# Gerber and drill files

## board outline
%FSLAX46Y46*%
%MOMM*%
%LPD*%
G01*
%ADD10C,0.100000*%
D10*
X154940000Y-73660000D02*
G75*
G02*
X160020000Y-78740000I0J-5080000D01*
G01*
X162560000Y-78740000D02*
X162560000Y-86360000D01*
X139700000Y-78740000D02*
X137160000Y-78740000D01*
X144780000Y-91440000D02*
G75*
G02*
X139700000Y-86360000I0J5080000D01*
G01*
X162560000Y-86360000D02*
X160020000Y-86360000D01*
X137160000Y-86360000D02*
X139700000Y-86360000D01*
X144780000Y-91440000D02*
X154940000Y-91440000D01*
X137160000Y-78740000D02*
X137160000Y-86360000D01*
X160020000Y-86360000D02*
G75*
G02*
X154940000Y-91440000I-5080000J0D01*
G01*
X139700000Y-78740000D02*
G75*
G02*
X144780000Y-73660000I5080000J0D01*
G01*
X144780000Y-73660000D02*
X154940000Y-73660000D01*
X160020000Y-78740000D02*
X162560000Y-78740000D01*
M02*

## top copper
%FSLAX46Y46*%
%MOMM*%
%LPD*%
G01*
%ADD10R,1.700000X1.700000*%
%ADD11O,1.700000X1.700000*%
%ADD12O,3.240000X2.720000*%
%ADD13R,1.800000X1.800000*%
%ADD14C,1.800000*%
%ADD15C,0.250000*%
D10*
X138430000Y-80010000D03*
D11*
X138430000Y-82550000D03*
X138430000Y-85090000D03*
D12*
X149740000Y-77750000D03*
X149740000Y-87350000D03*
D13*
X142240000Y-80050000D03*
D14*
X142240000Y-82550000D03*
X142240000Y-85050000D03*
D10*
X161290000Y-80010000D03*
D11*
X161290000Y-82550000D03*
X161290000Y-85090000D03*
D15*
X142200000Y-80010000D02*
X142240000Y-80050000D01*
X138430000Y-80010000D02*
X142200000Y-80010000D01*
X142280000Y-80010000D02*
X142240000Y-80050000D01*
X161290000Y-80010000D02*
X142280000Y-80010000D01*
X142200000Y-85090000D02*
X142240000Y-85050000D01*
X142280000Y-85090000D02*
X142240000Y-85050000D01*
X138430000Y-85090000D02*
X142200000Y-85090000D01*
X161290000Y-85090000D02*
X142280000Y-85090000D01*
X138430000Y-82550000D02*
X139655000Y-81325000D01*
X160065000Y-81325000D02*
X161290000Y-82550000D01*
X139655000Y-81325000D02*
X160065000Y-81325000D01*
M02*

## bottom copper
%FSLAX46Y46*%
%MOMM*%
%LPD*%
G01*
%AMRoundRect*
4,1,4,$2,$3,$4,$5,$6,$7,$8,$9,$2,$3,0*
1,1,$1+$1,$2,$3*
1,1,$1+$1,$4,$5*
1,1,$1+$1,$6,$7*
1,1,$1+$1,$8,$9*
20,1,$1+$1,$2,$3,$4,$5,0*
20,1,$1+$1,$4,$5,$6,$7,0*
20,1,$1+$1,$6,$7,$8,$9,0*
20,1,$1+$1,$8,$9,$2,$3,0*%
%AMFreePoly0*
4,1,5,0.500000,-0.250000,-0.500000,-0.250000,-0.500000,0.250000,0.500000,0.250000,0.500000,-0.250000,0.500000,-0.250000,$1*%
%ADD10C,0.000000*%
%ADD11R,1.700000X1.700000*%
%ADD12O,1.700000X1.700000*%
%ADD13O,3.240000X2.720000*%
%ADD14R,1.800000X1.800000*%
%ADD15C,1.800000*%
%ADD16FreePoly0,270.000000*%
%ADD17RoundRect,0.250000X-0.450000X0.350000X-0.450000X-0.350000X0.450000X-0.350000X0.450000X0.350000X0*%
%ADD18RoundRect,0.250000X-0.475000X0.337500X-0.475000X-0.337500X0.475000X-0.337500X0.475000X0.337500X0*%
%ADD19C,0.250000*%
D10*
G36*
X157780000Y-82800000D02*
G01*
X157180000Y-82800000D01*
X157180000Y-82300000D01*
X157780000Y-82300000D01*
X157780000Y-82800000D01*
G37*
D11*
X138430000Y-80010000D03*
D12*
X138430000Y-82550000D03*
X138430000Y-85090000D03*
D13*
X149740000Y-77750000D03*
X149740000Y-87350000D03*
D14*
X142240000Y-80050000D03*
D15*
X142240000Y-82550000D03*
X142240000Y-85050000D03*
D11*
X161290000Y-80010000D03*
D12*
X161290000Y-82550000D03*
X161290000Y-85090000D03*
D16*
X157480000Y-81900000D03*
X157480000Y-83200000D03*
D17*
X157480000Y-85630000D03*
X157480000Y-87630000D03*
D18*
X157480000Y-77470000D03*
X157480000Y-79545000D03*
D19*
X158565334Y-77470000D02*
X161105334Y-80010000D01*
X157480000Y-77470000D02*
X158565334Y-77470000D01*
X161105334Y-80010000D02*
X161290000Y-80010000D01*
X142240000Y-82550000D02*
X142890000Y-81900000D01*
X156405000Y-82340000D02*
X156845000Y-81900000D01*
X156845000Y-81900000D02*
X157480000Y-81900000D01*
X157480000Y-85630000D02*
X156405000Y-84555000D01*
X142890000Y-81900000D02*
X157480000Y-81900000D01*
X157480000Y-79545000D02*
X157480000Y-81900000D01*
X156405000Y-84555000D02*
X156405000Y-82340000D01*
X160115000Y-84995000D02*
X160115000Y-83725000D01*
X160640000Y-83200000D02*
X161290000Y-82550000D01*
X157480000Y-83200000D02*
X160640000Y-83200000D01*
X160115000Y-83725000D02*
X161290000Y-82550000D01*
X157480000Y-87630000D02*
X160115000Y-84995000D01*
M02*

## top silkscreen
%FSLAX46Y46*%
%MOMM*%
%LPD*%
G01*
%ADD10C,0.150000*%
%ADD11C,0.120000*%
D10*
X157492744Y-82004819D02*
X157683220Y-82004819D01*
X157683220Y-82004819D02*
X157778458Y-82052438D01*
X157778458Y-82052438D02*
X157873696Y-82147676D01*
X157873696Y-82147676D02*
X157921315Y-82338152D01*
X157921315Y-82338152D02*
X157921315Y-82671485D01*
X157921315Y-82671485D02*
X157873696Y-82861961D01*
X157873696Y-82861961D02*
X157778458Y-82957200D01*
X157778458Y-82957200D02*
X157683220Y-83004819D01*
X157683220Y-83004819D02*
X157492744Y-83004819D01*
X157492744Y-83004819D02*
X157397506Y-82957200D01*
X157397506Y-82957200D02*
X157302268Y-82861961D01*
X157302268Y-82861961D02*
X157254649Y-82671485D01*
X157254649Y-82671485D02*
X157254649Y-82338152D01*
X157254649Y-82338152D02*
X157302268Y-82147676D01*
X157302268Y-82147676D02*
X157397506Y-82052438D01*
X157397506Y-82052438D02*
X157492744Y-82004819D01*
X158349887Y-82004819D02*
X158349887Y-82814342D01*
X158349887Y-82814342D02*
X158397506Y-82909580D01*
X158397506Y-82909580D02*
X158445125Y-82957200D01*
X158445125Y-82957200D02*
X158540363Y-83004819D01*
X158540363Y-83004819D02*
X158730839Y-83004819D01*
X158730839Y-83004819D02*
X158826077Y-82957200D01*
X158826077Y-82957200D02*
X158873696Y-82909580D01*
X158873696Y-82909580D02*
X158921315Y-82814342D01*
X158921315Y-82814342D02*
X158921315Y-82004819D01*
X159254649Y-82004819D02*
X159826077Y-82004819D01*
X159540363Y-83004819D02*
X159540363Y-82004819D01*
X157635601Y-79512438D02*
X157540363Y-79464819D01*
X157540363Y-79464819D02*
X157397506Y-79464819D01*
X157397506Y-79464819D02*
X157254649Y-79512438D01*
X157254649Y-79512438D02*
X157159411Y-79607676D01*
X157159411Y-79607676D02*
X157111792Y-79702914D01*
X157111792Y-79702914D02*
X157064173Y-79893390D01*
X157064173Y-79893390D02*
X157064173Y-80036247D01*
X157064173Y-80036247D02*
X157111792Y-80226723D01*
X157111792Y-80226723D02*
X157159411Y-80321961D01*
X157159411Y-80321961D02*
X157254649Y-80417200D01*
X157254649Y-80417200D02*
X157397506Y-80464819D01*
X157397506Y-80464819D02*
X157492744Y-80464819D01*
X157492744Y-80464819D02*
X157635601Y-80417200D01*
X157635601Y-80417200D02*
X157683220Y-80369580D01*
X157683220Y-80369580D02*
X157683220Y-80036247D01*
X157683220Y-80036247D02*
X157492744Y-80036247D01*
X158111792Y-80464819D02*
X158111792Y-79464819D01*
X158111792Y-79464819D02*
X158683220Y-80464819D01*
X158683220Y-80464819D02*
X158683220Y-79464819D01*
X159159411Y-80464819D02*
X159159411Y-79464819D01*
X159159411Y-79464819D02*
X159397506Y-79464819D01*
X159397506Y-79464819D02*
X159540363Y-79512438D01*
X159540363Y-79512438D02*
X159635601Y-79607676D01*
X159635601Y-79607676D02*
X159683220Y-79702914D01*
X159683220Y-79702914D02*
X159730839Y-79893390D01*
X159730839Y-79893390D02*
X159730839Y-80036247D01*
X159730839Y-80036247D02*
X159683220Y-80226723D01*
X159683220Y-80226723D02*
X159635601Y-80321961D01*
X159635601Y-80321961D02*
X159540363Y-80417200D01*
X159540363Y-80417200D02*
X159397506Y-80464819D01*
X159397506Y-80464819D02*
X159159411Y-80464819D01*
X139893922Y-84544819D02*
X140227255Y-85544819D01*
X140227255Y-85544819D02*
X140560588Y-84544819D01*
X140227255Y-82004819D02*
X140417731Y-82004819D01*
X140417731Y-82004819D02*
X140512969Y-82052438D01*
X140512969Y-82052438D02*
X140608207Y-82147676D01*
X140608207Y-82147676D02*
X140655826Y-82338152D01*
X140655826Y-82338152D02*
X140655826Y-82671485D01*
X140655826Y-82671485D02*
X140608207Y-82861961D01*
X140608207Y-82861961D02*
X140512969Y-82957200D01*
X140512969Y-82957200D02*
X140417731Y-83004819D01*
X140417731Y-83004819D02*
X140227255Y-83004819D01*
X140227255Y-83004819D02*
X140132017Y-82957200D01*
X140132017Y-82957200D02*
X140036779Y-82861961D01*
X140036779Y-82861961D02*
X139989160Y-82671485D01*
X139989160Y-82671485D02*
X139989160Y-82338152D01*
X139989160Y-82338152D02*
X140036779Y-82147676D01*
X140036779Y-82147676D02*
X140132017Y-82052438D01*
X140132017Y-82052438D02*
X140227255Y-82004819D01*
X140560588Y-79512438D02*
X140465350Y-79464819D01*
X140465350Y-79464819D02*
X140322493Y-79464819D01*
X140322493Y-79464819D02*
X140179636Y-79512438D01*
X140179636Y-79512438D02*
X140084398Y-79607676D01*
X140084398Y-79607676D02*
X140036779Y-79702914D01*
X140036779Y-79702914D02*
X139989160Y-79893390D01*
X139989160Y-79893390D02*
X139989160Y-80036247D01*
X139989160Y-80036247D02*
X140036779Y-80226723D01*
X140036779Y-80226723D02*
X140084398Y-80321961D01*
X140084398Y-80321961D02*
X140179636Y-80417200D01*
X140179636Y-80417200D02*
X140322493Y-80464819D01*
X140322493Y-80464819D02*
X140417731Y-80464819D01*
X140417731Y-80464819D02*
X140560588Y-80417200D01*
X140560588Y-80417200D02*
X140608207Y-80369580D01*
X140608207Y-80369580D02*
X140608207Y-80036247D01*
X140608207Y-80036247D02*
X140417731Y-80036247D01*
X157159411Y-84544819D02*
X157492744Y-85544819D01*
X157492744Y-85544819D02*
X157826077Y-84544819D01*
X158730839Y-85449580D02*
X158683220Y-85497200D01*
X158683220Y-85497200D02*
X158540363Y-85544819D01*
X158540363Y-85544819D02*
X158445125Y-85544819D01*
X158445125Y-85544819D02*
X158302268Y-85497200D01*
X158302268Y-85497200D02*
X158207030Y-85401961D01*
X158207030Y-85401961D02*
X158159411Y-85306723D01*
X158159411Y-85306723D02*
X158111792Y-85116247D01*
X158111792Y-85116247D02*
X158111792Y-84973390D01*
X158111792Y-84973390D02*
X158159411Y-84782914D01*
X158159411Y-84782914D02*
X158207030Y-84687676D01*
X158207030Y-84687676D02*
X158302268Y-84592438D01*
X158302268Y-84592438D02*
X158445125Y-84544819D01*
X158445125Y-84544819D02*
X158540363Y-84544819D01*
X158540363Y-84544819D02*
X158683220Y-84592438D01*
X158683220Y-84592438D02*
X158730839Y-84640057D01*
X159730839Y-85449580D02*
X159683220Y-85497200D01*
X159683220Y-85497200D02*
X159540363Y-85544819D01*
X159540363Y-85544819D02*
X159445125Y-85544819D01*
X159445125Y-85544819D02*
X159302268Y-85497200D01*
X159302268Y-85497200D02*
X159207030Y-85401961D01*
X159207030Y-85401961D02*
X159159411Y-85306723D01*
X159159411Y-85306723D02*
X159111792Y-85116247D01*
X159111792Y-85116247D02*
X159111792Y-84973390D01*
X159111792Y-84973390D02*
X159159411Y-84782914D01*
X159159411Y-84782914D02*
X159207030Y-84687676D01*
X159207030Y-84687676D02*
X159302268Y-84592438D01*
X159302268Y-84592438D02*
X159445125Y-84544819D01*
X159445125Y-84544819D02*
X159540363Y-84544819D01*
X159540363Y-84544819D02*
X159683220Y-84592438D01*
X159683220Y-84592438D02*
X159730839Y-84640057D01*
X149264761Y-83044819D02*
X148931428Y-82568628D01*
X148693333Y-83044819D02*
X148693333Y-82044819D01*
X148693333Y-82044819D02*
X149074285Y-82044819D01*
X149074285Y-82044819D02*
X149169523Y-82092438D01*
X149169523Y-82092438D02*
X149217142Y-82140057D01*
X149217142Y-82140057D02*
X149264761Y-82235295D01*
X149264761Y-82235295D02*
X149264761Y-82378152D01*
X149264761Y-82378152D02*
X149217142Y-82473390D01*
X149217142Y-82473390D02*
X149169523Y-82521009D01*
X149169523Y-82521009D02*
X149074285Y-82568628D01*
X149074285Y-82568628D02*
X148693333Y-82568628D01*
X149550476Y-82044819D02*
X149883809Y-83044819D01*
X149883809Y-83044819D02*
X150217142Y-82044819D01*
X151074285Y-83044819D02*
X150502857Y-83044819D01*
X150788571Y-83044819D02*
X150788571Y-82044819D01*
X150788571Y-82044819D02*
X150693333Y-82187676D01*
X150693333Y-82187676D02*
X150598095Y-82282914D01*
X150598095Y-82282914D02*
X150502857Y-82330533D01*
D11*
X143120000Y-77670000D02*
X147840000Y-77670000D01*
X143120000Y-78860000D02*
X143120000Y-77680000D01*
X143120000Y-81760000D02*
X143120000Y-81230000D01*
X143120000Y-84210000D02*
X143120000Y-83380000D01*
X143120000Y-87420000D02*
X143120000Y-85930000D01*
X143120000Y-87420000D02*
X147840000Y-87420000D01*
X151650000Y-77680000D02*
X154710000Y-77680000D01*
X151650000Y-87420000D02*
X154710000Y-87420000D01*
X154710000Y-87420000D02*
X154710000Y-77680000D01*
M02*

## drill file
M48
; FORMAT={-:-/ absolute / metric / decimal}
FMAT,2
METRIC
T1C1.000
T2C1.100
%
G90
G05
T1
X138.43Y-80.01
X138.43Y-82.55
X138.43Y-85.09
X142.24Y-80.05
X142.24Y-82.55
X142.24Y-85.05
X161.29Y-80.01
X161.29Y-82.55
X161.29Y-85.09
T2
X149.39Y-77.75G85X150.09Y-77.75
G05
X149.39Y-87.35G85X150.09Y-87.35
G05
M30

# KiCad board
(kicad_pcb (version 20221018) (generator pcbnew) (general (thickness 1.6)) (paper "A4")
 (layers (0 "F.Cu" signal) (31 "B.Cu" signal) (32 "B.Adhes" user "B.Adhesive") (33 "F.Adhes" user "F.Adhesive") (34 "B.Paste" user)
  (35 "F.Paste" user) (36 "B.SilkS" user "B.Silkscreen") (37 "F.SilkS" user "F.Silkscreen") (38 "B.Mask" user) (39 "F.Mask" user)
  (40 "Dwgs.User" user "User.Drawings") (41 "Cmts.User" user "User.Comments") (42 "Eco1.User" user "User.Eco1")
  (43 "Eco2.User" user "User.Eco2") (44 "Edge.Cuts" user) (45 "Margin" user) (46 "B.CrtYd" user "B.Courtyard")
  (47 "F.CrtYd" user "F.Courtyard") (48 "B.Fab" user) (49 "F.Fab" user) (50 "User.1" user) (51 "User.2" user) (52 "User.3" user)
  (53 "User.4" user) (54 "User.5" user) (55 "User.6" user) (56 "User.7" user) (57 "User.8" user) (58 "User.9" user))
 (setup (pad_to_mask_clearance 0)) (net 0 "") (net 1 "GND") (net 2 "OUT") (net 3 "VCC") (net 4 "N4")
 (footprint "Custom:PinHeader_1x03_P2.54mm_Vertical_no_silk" (layer "F.Cu") (at 138.43 80.01)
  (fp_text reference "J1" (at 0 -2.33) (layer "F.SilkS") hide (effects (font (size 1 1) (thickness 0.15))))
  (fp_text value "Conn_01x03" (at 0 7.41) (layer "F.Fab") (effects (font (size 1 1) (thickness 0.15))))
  (pad "1" thru_hole rect (at 0 0) (size 1.7 1.7) (drill 1) (layers "*.Cu" "*.Mask") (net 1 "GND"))
  (pad "2" thru_hole oval (at 0 2.54) (size 1.7 1.7) (drill 1) (layers "*.Cu" "*.Mask") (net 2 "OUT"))
  (pad "3" thru_hole oval (at 0 5.08) (size 1.7 1.7) (drill 1) (layers "*.Cu" "*.Mask") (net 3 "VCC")))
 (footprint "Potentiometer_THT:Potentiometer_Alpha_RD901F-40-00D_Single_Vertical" (layer "F.Cu") (at 142.24 80.05)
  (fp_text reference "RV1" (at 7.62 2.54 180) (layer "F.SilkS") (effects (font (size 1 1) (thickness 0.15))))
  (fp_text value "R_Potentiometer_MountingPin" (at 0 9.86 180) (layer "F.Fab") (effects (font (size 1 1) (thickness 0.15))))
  (fp_line (start 0.88 -2.38) (end 5.6 -2.38) (stroke (width 0.12) (type solid)) (layer "F.SilkS"))
  (fp_line (start 0.88 -1.19) (end 0.88 -2.37) (stroke (width 0.12) (type solid)) (layer "F.SilkS"))
  (fp_line (start 0.88 1.71) (end 0.88 1.18) (stroke (width 0.12) (type solid)) (layer "F.SilkS"))
  (fp_line (start 0.88 4.16) (end 0.88 3.33) (stroke (width 0.12) (type solid)) (layer "F.SilkS"))
  (fp_line (start 0.88 7.37) (end 0.88 5.88) (stroke (width 0.12) (type solid)) (layer "F.SilkS"))
  (fp_line (start 0.88 7.37) (end 5.6 7.37) (stroke (width 0.12) (type solid)) (layer "F.SilkS"))
  (fp_line (start 9.41 -2.37) (end 12.47 -2.37) (stroke (width 0.12) (type solid)) (layer "F.SilkS"))
  (fp_line (start 9.41 7.37) (end 12.47 7.37) (stroke (width 0.12) (type solid)) (layer "F.SilkS"))
  (fp_line (start 12.47 7.37) (end 12.47 -2.37) (stroke (width 0.12) (type solid)) (layer "F.SilkS"))
  (pad "" thru_hole oval (at 7.5 -2.3 90) (size 2.72 3.24) (drill oval 1.1 1.8) (layers "*.Cu" "*.Mask"))
  (pad "" thru_hole oval (at 7.5 7.3 90) (size 2.72 3.24) (drill oval 1.1 1.8) (layers "*.Cu" "*.Mask"))
  (pad "1" thru_hole rect (at 0 0 90) (size 1.8 1.8) (drill 1) (layers "*.Cu" "*.Mask") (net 1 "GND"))
  (pad "2" thru_hole circle (at 0 2.5 90) (size 1.8 1.8) (drill 1) (layers "*.Cu" "*.Mask") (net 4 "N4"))
  (pad "3" thru_hole circle (at 0 5 90) (size 1.8 1.8) (drill 1) (layers "*.Cu" "*.Mask") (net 3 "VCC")))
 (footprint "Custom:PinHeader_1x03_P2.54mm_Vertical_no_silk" (layer "F.Cu") (at 161.29 80.01)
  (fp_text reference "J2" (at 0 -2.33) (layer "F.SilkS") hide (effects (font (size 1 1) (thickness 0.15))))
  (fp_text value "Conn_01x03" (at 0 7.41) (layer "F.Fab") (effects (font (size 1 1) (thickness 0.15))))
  (pad "1" thru_hole rect (at 0 0) (size 1.7 1.7) (drill 1) (layers "*.Cu" "*.Mask") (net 1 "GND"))
  (pad "2" thru_hole oval (at 0 2.54) (size 1.7 1.7) (drill 1) (layers "*.Cu" "*.Mask") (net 2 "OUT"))
  (pad "3" thru_hole oval (at 0 5.08) (size 1.7 1.7) (drill 1) (layers "*.Cu" "*.Mask") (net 3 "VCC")))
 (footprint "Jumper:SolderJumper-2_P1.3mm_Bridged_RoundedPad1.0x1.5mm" (layer "B.Cu") (at 157.48 82.55 -90) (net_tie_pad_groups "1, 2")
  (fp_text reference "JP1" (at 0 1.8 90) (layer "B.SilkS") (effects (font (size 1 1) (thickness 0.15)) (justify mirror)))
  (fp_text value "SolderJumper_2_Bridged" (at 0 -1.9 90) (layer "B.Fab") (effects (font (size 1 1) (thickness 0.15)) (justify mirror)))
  (fp_poly (pts (xy 0.25 0.3) (xy -0.25 0.3) (xy -0.25 -0.3) (xy 0.25 -0.3)) (stroke (width 0) (type solid)) (fill solid) (layer "B.Cu"))
  (pad "1" smd custom (at -0.65 0 270) (size 1 0.5) (layers "B.Cu" "B.Mask") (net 4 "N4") (zone_connect 2) (thermal_bridge_angle 45)
   (options (clearance outline) (anchor rect)) (primitives))
  (pad "2" smd custom (at 0.65 0 270) (size 1 0.5) (layers "B.Cu" "B.Mask") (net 2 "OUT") (zone_connect 2) (thermal_bridge_angle 45)
   (options (clearance outline) (anchor rect)) (primitives)))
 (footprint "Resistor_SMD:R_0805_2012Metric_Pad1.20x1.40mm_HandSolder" (layer "B.Cu") (at 157.48 86.63 -90)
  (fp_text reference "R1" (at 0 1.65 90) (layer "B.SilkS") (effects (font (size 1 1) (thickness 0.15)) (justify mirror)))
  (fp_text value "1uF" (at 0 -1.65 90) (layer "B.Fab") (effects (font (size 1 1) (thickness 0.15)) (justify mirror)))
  (pad "1" smd roundrect (at -1 0 270) (size 1.2 1.4) (layers "B.Cu" "B.Paste" "B.Mask") (roundrect_rratio 0.208333) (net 4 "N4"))
  (pad "2" smd roundrect (at 1 0 270) (size 1.2 1.4) (layers "B.Cu" "B.Paste" "B.Mask") (roundrect_rratio 0.208333) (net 2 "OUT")))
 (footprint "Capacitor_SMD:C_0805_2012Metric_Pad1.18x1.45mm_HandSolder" (layer "B.Cu") (at 157.48 78.5075 -90)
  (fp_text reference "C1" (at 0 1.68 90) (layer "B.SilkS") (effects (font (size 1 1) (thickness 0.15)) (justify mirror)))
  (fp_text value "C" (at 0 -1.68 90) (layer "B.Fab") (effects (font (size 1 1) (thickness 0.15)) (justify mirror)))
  (pad "1" smd roundrect (at -1.0375 0 270) (size 1.175 1.45) (layers "B.Cu" "B.Paste" "B.Mask") (roundrect_rratio 0.212766) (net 1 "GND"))
  (pad "2" smd roundrect (at 1.0375 0 270) (size 1.175 1.45) (layers "B.Cu" "B.Paste" "B.Mask") (roundrect_rratio 0.212766) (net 4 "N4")))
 (gr_arc (start 154.94 73.66) (mid 158.532102 75.147898) (end 160.02 78.74) (stroke (width 0.1) (type default)) (layer "Edge.Cuts"))
 (gr_line (start 162.56 78.74) (end 162.56 86.36) (stroke (width 0.1) (type default)) (layer "Edge.Cuts"))
 (gr_line (start 139.7 78.74) (end 137.16 78.74) (stroke (width 0.1) (type default)) (layer "Edge.Cuts"))
 (gr_arc (start 144.78 91.44) (mid 141.187898 89.952102) (end 139.7 86.36) (stroke (width 0.1) (type default)) (layer "Edge.Cuts"))
 (gr_line (start 162.56 86.36) (end 160.02 86.36) (stroke (width 0.1) (type default)) (layer "Edge.Cuts"))
 (gr_line (start 137.16 86.36) (end 139.7 86.36) (stroke (width 0.1) (type default)) (layer "Edge.Cuts"))
 (gr_line (start 144.78 91.44) (end 154.94 91.44) (stroke (width 0.1) (type default)) (layer "Edge.Cuts"))
 (gr_line (start 137.16 78.74) (end 137.16 86.36) (stroke (width 0.1) (type default)) (layer "Edge.Cuts"))
 (gr_arc (start 160.02 86.36) (mid 158.532102 89.952102) (end 154.94 91.44) (stroke (width 0.1) (type default)) (layer "Edge.Cuts"))
 (gr_arc (start 139.7 78.74) (mid 141.187898 75.147898) (end 144.78 73.66) (stroke (width 0.1) (type default)) (layer "Edge.Cuts"))
 (gr_line (start 144.78 73.66) (end 154.94 73.66) (stroke (width 0.1) (type default)) (layer "Edge.Cuts"))
 (gr_line (start 160.02 78.74) (end 162.56 78.74) (stroke (width 0.1) (type default)) (layer "Edge.Cuts"))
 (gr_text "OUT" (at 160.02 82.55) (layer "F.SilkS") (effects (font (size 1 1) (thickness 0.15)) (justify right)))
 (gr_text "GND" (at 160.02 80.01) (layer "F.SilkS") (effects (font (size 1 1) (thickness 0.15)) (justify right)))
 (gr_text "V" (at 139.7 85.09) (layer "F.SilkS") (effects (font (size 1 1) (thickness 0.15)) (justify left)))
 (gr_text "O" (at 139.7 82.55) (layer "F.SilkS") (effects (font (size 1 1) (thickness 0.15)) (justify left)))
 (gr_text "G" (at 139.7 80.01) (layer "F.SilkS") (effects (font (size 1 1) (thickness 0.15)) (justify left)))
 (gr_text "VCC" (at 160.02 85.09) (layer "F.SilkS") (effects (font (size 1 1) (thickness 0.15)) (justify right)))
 (segment (start 142.2 80.01) (end 142.24 80.05) (width 0.25) (layer "F.Cu") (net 1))
 (segment (start 138.43 80.01) (end 142.2 80.01) (width 0.25) (layer "F.Cu") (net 1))
 (segment (start 142.28 80.01) (end 142.24 80.05) (width 0.25) (layer "F.Cu") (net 1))
 (segment (start 161.29 80.01) (end 142.28 80.01) (width 0.25) (layer "F.Cu") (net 1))
 (segment (start 158.565334 77.47) (end 161.105334 80.01) (width 0.25) (layer "B.Cu") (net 1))
 (segment (start 157.48 77.47) (end 158.565334 77.47) (width 0.25) (layer "B.Cu") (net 1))
 (segment (start 161.105334 80.01) (end 161.29 80.01) (width 0.25) (layer "B.Cu") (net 1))
 (segment (start 142.24 82.55) (end 142.89 81.9) (width 0.25) (layer "B.Cu") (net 4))
 (segment (start 156.405 82.34) (end 156.845 81.9) (width 0.25) (layer "B.Cu") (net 4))
 (segment (start 156.845 81.9) (end 157.48 81.9) (width 0.25) (layer "B.Cu") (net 4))
 (segment (start 157.48 85.63) (end 156.405 84.555) (width 0.25) (layer "B.Cu") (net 4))
 (segment (start 142.89 81.9) (end 157.48 81.9) (width 0.25) (layer "B.Cu") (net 4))
 (segment (start 157.48 79.545) (end 157.48 81.9) (width 0.25) (layer "B.Cu") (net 4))
 (segment (start 156.405 84.555) (end 156.405 82.34) (width 0.25) (layer "B.Cu") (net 4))
 (segment (start 142.2 85.09) (end 142.24 85.05) (width 0.25) (layer "F.Cu") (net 3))
 (segment (start 142.28 85.09) (end 142.24 85.05) (width 0.25) (layer "F.Cu") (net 3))
 (segment (start 138.43 85.09) (end 142.2 85.09) (width 0.25) (layer "F.Cu") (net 3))
 (segment (start 161.29 85.09) (end 142.28 85.09) (width 0.25) (layer "F.Cu") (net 3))
 (segment (start 138.43 82.55) (end 139.655 81.325) (width 0.25) (layer "F.Cu") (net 2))
 (segment (start 160.065 81.325) (end 161.29 82.55) (width 0.25) (layer "F.Cu") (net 2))
 (segment (start 139.655 81.325) (end 160.065 81.325) (width 0.25) (layer "F.Cu") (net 2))
 (segment (start 160.115 84.995) (end 160.115 83.725) (width 0.25) (layer "B.Cu") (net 2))
 (segment (start 160.64 83.2) (end 161.29 82.55) (width 0.25) (layer "B.Cu") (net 2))
 (segment (start 157.48 83.2) (end 160.64 83.2) (width 0.25) (layer "B.Cu") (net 2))
 (segment (start 160.115 83.725) (end 161.29 82.55) (width 0.25) (layer "B.Cu") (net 2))
 (segment (start 157.48 87.63) (end 160.115 84.995) (width 0.25) (layer "B.Cu") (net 2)))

